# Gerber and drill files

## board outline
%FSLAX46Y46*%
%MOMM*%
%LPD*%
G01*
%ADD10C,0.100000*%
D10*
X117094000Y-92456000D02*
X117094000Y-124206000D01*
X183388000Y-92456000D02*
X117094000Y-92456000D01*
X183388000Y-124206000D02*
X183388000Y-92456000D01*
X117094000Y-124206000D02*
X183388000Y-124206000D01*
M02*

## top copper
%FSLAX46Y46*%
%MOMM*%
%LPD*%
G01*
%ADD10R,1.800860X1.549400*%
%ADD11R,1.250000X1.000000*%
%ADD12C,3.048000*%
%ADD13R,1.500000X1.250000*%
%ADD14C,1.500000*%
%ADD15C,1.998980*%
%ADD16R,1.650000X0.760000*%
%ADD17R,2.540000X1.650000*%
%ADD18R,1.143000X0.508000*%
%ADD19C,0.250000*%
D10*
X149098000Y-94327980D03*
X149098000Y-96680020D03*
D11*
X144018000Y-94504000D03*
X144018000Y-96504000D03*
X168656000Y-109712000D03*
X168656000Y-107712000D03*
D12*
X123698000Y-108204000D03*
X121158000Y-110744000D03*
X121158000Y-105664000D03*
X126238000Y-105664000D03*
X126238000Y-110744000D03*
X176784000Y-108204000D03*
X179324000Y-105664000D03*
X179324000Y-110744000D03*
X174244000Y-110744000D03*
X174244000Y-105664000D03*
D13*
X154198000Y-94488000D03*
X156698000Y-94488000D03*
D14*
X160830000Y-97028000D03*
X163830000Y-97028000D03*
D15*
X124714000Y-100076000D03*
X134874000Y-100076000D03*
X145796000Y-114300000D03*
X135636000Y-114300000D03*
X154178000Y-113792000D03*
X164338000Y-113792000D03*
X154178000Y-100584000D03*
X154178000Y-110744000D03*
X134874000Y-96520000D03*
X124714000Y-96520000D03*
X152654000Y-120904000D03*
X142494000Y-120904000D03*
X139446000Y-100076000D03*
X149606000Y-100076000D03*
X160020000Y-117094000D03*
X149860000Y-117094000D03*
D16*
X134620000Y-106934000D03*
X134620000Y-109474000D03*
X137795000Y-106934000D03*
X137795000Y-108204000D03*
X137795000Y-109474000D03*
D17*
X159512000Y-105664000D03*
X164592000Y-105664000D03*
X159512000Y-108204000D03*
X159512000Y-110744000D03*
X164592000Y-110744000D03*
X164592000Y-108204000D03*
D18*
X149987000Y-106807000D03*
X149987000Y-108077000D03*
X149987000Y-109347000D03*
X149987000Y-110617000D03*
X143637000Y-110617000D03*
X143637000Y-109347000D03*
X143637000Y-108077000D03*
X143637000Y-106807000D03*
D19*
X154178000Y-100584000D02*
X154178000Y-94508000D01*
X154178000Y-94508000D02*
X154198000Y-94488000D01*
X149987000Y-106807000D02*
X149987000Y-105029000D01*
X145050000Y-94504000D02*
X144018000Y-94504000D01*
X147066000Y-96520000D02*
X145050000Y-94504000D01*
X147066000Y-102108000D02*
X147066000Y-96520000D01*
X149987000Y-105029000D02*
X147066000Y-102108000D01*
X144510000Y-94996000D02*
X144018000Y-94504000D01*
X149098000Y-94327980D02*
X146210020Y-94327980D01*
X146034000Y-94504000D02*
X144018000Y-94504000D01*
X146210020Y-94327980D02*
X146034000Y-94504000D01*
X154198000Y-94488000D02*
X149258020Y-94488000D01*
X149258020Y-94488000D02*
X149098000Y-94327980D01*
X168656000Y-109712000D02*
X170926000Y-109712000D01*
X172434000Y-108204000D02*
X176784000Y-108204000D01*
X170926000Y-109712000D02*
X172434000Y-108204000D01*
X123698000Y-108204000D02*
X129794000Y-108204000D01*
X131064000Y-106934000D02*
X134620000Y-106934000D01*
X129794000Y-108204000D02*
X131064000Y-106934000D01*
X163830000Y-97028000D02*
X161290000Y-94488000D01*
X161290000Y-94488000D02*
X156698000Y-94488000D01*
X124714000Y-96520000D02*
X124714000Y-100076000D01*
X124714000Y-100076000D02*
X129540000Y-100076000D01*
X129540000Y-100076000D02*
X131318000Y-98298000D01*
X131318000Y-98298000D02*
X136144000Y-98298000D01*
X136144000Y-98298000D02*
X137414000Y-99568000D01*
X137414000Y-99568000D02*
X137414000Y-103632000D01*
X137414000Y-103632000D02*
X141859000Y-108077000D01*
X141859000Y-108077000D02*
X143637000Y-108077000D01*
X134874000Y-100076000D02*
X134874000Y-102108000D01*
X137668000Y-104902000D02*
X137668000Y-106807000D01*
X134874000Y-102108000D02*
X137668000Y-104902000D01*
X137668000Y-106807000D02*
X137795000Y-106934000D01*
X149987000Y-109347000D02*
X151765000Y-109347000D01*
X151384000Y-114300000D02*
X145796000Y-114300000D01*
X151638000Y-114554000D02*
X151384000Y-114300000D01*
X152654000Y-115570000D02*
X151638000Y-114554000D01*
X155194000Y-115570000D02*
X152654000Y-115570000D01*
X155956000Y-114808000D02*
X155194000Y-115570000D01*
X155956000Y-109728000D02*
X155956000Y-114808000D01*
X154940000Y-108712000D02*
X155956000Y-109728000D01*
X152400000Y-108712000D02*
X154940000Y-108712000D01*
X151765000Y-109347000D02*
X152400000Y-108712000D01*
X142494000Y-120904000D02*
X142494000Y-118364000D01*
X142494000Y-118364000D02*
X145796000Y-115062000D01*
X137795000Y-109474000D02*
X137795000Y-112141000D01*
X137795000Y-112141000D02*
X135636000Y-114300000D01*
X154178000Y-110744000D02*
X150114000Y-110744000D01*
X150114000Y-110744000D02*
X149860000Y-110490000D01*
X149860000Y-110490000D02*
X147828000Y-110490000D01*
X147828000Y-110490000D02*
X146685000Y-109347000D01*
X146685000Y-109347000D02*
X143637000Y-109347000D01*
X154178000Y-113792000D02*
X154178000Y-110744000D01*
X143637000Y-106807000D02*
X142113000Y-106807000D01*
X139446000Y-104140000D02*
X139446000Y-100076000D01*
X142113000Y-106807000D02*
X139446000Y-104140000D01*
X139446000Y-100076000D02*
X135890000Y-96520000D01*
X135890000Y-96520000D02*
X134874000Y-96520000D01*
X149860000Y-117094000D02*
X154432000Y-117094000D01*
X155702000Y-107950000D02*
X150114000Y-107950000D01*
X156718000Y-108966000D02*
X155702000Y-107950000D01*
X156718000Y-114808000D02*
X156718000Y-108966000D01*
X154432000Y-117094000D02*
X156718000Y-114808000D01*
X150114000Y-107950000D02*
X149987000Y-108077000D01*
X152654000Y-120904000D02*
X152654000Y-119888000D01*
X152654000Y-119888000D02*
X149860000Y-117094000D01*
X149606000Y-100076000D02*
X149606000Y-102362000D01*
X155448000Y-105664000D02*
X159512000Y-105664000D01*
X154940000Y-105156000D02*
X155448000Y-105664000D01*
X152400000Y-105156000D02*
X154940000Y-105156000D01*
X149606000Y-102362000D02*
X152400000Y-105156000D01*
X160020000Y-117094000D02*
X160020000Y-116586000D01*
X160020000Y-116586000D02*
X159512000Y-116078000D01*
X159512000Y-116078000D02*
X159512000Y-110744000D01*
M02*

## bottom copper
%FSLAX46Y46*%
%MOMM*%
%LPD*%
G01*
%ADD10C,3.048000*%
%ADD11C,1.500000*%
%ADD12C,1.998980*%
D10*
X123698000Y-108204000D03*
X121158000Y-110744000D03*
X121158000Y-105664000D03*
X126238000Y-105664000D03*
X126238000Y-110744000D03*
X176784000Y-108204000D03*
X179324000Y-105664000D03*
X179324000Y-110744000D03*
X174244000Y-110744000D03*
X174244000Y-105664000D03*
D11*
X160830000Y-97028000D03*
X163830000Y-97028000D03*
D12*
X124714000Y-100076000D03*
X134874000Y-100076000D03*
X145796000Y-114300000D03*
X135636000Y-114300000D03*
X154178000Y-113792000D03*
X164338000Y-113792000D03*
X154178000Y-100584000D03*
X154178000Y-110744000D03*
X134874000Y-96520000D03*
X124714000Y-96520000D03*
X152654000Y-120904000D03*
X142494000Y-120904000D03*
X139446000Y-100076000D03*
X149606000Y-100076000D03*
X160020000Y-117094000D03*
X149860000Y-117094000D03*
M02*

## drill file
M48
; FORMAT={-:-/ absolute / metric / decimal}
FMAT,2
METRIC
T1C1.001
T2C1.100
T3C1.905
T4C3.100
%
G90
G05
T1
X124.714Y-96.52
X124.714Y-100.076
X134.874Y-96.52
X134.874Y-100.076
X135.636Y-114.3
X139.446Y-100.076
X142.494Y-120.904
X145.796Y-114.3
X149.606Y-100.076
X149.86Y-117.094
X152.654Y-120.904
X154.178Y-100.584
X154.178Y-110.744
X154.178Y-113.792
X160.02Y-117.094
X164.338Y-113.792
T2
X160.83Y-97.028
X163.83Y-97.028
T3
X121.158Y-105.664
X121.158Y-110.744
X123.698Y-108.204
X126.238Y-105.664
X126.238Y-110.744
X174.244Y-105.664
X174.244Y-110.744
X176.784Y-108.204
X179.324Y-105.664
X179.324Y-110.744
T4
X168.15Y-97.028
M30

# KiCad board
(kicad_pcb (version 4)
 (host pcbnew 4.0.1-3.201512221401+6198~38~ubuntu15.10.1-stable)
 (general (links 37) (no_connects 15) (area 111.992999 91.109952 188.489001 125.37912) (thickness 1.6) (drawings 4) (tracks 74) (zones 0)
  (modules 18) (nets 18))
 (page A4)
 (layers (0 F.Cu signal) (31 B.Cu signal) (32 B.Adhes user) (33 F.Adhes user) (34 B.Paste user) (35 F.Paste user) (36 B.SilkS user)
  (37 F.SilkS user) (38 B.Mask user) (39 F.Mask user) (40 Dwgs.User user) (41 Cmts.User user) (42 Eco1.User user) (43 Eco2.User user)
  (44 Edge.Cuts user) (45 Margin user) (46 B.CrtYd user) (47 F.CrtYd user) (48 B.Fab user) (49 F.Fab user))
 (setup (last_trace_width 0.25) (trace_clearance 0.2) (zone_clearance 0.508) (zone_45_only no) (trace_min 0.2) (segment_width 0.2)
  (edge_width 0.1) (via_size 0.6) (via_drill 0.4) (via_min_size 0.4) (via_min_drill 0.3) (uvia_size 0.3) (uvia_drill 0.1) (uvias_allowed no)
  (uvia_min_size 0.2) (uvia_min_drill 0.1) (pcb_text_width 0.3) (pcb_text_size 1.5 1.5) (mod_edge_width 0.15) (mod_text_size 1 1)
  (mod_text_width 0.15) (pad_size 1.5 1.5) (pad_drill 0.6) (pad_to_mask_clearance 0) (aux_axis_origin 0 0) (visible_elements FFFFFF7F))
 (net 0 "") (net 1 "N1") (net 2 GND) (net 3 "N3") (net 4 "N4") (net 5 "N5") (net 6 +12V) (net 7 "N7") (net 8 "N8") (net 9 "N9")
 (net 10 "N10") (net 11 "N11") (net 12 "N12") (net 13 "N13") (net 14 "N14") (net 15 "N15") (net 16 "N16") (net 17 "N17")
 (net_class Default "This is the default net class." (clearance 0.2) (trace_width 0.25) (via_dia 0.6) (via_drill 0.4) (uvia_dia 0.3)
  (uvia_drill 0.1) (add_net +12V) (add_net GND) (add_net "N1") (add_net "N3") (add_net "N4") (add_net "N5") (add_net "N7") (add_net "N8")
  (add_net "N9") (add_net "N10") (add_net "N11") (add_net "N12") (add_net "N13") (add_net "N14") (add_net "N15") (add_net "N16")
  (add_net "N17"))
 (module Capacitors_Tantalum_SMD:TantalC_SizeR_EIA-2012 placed (layer F.Cu) (at 149.098 95.504 90)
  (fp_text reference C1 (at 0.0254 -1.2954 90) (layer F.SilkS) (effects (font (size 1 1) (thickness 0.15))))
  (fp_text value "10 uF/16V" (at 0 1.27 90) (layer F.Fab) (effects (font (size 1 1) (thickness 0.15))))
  (pad 1 smd rect (at 1.17602 0 90) (size 1.5494 1.80086) (layers F.Cu F.Paste F.Mask) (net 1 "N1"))
  (pad 2 smd rect (at -1.17602 0 90) (size 1.5494 1.80086) (layers F.Cu F.Paste F.Mask) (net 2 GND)))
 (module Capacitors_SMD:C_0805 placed (layer F.Cu) (at 144.018 95.504 270)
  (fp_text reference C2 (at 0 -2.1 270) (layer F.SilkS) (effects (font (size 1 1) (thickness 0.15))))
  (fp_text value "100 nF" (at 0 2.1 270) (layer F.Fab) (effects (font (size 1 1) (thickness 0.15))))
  (pad 1 smd rect (at -1 0 270) (size 1 1.25) (layers F.Cu F.Paste F.Mask) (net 1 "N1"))
  (pad 2 smd rect (at 1 0 270) (size 1 1.25) (layers F.Cu F.Paste F.Mask) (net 2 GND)))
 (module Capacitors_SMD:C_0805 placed (layer F.Cu) (at 168.656 108.712 90)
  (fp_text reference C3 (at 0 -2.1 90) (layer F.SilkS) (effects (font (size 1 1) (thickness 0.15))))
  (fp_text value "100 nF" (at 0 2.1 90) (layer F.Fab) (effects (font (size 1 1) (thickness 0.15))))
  (pad 1 smd rect (at -1 0 90) (size 1 1.25) (layers F.Cu F.Paste F.Mask) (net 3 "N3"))
  (pad 2 smd rect (at 1 0 90) (size 1 1.25) (layers F.Cu F.Paste F.Mask) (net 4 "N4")))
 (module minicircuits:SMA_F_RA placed (layer F.Cu) (at 123.698 108.204 180)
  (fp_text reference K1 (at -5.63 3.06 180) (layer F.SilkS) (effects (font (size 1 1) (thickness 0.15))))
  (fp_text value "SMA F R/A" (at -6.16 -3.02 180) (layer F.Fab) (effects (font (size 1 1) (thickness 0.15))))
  (pad 1 thru_hole circle (at 0 0 180) (size 3.048 3.048) (drill 1.905) (layers *.Cu *.Mask F.SilkS) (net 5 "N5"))
  (pad 2 thru_hole circle (at 2.54 -2.54 180) (size 3.048 3.048) (drill 1.905) (layers *.Cu *.Mask F.SilkS) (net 2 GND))
  (pad 3 thru_hole circle (at 2.54 2.54 180) (size 3.048 3.048) (drill 1.905) (layers *.Cu *.Mask F.SilkS) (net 2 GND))
  (pad 4 thru_hole circle (at -2.54 2.54 180) (size 3.048 3.048) (drill 1.905) (layers *.Cu *.Mask F.SilkS) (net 2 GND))
  (pad 5 thru_hole circle (at -2.54 -2.54 180) (size 3.048 3.048) (drill 1.905) (layers *.Cu *.Mask F.SilkS) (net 2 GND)))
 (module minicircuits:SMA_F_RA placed (layer F.Cu) (at 176.784 108.204)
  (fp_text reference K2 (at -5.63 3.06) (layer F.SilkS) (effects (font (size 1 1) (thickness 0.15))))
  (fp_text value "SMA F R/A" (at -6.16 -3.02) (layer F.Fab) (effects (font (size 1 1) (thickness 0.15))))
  (pad 1 thru_hole circle (at 0 0) (size 3.048 3.048) (drill 1.905) (layers *.Cu *.Mask F.SilkS) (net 3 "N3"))
  (pad 2 thru_hole circle (at 2.54 -2.54) (size 3.048 3.048) (drill 1.905) (layers *.Cu *.Mask F.SilkS) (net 2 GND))
  (pad 3 thru_hole circle (at 2.54 2.54) (size 3.048 3.048) (drill 1.905) (layers *.Cu *.Mask F.SilkS) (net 2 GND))
  (pad 4 thru_hole circle (at -2.54 2.54) (size 3.048 3.048) (drill 1.905) (layers *.Cu *.Mask F.SilkS) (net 2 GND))
  (pad 5 thru_hole circle (at -2.54 -2.54) (size 3.048 3.048) (drill 1.905) (layers *.Cu *.Mask F.SilkS) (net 2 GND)))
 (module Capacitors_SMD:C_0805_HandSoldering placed (layer F.Cu) (at 155.448 94.488)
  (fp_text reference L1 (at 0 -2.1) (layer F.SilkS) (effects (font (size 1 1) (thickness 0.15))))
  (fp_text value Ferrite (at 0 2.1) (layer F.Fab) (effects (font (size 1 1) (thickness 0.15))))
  (pad 1 smd rect (at -1.25 0) (size 1.5 1.25) (layers F.Cu F.Paste F.Mask) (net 1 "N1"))
  (pad 2 smd rect (at 1.25 0) (size 1.5 1.25) (layers F.Cu F.Paste F.Mask) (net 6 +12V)))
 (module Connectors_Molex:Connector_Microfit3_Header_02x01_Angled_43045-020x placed (layer F.Cu) (at 163.83 97.028 90)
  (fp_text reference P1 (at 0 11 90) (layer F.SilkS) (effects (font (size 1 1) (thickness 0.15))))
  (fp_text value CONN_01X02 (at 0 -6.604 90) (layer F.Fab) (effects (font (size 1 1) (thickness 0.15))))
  (pad 2 thru_hole circle (at 0 -3 90) (size 1.5 1.5) (drill 1.1) (layers *.Cu *.Mask F.SilkS) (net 2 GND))
  (pad 1 thru_hole circle (at 0 0 90) (size 1.5 1.5) (drill 1.1) (layers *.Cu *.Mask F.SilkS) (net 6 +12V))
  (pad "" np_thru_hole circle (at 0 4.32 90) (size 3.1 3.1) (drill 3.1) (layers *.Cu *.Mask F.SilkS)))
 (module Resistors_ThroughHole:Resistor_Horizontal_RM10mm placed (layer F.Cu) (at 129.794 100.076)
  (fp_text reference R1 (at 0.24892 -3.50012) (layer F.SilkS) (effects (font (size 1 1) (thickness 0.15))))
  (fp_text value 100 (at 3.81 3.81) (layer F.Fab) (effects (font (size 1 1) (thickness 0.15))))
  (pad 1 thru_hole circle (at -5.08 0) (size 1.99898 1.99898) (drill 1.00076) (layers *.Cu *.SilkS *.Mask) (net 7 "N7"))
  (pad 2 thru_hole circle (at 5.08 0) (size 1.99898 1.99898) (drill 1.00076) (layers *.Cu *.SilkS *.Mask) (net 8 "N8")))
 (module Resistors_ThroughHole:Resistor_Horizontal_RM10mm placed (layer F.Cu) (at 140.716 114.3 180)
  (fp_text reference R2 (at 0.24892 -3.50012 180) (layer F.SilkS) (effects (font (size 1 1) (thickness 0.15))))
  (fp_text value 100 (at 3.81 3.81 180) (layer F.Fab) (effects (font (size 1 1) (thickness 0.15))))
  (pad 1 thru_hole circle (at -5.08 0 180) (size 1.99898 1.99898) (drill 1.00076) (layers *.Cu *.SilkS *.Mask) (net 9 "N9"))
  (pad 2 thru_hole circle (at 5.08 0 180) (size 1.99898 1.99898) (drill 1.00076) (layers *.Cu *.SilkS *.Mask) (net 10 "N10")))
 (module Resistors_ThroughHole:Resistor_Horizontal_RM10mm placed (layer F.Cu) (at 159.258 113.792)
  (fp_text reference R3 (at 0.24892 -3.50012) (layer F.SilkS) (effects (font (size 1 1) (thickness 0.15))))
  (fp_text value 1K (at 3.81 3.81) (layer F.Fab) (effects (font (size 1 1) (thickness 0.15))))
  (pad 1 thru_hole circle (at -5.08 0) (size 1.99898 1.99898) (drill 1.00076) (layers *.Cu *.SilkS *.Mask) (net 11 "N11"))
  (pad 2 thru_hole circle (at 5.08 0) (size 1.99898 1.99898) (drill 1.00076) (layers *.Cu *.SilkS *.Mask) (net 2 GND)))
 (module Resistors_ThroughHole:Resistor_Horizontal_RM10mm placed (layer F.Cu) (at 154.178 105.664 270)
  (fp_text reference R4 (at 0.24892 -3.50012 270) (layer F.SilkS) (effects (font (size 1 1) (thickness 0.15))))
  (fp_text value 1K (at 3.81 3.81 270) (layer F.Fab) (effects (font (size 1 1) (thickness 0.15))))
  (pad 1 thru_hole circle (at -5.08 0 270) (size 1.99898 1.99898) (drill 1.00076) (layers *.Cu *.SilkS *.Mask) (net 1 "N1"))
  (pad 2 thru_hole circle (at 5.08 0 270) (size 1.99898 1.99898) (drill 1.00076) (layers *.Cu *.SilkS *.Mask) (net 11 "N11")))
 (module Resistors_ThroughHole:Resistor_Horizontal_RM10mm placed (layer F.Cu) (at 129.794 96.52 180)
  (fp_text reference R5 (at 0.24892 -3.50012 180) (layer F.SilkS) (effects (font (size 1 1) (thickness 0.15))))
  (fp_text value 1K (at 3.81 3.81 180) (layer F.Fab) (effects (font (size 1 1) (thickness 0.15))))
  (pad 1 thru_hole circle (at -5.08 0 180) (size 1.99898 1.99898) (drill 1.00076) (layers *.Cu *.SilkS *.Mask) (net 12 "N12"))
  (pad 2 thru_hole circle (at 5.08 0 180) (size 1.99898 1.99898) (drill 1.00076) (layers *.Cu *.SilkS *.Mask) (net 7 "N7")))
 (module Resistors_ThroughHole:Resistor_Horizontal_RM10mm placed (layer F.Cu) (at 147.574 120.904 180)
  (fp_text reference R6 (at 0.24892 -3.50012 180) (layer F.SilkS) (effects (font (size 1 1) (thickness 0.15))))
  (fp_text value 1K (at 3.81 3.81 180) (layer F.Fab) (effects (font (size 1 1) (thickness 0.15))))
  (pad 1 thru_hole circle (at -5.08 0 180) (size 1.99898 1.99898) (drill 1.00076) (layers *.Cu *.SilkS *.Mask) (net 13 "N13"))
  (pad 2 thru_hole circle (at 5.08 0 180) (size 1.99898 1.99898) (drill 1.00076) (layers *.Cu *.SilkS *.Mask) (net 9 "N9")))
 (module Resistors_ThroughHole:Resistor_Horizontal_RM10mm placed (layer F.Cu) (at 144.526 100.076)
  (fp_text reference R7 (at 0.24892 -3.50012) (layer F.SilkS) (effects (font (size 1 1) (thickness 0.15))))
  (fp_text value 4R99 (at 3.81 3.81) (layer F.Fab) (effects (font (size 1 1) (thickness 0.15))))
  (pad 1 thru_hole circle (at -5.08 0) (size 1.99898 1.99898) (drill 1.00076) (layers *.Cu *.SilkS *.Mask) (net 12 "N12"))
  (pad 2 thru_hole circle (at 5.08 0) (size 1.99898 1.99898) (drill 1.00076) (layers *.Cu *.SilkS *.Mask) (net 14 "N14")))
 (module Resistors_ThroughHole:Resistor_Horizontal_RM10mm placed (layer F.Cu) (at 154.94 117.094 180)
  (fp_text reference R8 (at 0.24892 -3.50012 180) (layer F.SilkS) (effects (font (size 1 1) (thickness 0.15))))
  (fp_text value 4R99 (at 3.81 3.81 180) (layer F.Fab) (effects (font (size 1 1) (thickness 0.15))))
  (pad 1 thru_hole circle (at -5.08 0 180) (size 1.99898 1.99898) (drill 1.00076) (layers *.Cu *.SilkS *.Mask) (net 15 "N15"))
  (pad 2 thru_hole circle (at 5.08 0 180) (size 1.99898 1.99898) (drill 1.00076) (layers *.Cu *.SilkS *.Mask) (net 13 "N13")))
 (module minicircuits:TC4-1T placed (layer F.Cu) (at 134.62 106.934 270)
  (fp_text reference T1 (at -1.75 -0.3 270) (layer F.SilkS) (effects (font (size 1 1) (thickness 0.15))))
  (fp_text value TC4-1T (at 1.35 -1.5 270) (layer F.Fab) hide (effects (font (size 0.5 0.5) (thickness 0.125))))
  (pad 5 smd rect (at 0 0 270) (size 0.76 1.65) (layers F.Cu F.Paste F.Mask) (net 5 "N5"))
  (pad 4 smd rect (at 2.54 0 270) (size 0.76 1.65) (layers F.Cu F.Paste F.Mask) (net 2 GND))
  (pad 1 smd rect (at 0 -3.175 270) (size 0.76 1.65) (layers F.Cu F.Paste F.Mask) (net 8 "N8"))
  (pad 2 smd rect (at 1.27 -3.175 270) (size 0.76 1.65) (layers F.Cu F.Paste F.Mask) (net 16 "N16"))
  (pad 3 smd rect (at 2.54 -3.175 270) (size 0.76 1.65) (layers F.Cu F.Paste F.Mask) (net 10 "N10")))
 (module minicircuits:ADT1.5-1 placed (layer F.Cu) (at 159.512 105.664 270)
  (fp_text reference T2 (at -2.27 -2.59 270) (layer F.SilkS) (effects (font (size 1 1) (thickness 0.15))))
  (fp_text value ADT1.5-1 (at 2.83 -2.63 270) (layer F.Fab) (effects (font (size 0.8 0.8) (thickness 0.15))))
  (pad 1 smd rect (at 0 0 270) (size 1.65 2.54) (layers F.Cu F.Paste F.Mask) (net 14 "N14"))
  (pad 6 smd rect (at 0 -5.08 270) (size 1.65 2.54) (layers F.Cu F.Paste F.Mask))
  (pad 2 smd rect (at 2.54 0 270) (size 1.65 2.54) (layers F.Cu F.Paste F.Mask) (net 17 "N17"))
  (pad 3 smd rect (at 5.08 0 270) (size 1.65 2.54) (layers F.Cu F.Paste F.Mask) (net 15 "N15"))
  (pad 4 smd rect (at 5.08 -5.08 270) (size 1.65 2.54) (layers F.Cu F.Paste F.Mask) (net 2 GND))
  (pad 5 smd rect (at 2.54 -5.08 270) (size 1.65 2.54) (layers F.Cu F.Paste F.Mask) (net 4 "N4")))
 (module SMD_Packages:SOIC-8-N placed (layer F.Cu) (at 146.812 108.712 270)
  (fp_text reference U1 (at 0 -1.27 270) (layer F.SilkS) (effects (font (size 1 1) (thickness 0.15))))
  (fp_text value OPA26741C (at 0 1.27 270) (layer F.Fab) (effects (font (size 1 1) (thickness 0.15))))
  (pad 8 smd rect (at -1.905 -3.175 270) (size 0.508 1.143) (layers F.Cu F.Paste F.Mask) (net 1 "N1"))
  (pad 7 smd rect (at -0.635 -3.175 270) (size 0.508 1.143) (layers F.Cu F.Paste F.Mask) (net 13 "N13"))
  (pad 6 smd rect (at 0.635 -3.175 270) (size 0.508 1.143) (layers F.Cu F.Paste F.Mask) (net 9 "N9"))
  (pad 5 smd rect (at 1.905 -3.175 270) (size 0.508 1.143) (layers F.Cu F.Paste F.Mask) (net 11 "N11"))
  (pad 4 smd rect (at 1.905 3.175 270) (size 0.508 1.143) (layers F.Cu F.Paste F.Mask) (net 2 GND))
  (pad 3 smd rect (at 0.635 3.175 270) (size 0.508 1.143) (layers F.Cu F.Paste F.Mask) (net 11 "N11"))
  (pad 2 smd rect (at -0.635 3.175 270) (size 0.508 1.143) (layers F.Cu F.Paste F.Mask) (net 7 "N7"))
  (pad 1 smd rect (at -1.905 3.175 270) (size 0.508 1.143) (layers F.Cu F.Paste F.Mask) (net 12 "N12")))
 (gr_line (start 117.094 92.456) (end 117.094 124.206) (angle 90) (layer Edge.Cuts) (width 0.1))
 (gr_line (start 183.388 92.456) (end 117.094 92.456) (angle 90) (layer Edge.Cuts) (width 0.1))
 (gr_line (start 183.388 124.206) (end 183.388 92.456) (angle 90) (layer Edge.Cuts) (width 0.1))
 (gr_line (start 117.094 124.206) (end 183.388 124.206) (angle 90) (layer Edge.Cuts) (width 0.1))
 (segment (start 154.178 100.584) (end 154.178 94.508) (width 0.25) (layer F.Cu) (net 1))
 (segment (start 154.178 94.508) (end 154.198 94.488) (width 0.25) (layer F.Cu) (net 1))
 (segment (start 149.987 106.807) (end 149.987 105.029) (width 0.25) (layer F.Cu) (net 1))
 (segment (start 145.05 94.504) (end 144.018 94.504) (width 0.25) (layer F.Cu) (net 1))
 (segment (start 147.066 96.52) (end 145.05 94.504) (width 0.25) (layer F.Cu) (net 1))
 (segment (start 147.066 102.108) (end 147.066 96.52) (width 0.25) (layer F.Cu) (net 1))
 (segment (start 149.987 105.029) (end 147.066 102.108) (width 0.25) (layer F.Cu) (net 1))
 (segment (start 144.51 94.996) (end 144.018 94.504) (width 0.25) (layer F.Cu) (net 1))
 (segment (start 149.098 94.32798) (end 146.21002 94.32798) (width 0.25) (layer F.Cu) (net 1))
 (segment (start 146.034 94.504) (end 144.018 94.504) (width 0.25) (layer F.Cu) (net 1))
 (segment (start 146.21002 94.32798) (end 146.034 94.504) (width 0.25) (layer F.Cu) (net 1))
 (segment (start 154.198 94.488) (end 149.25802 94.488) (width 0.25) (layer F.Cu) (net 1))
 (segment (start 149.25802 94.488) (end 149.098 94.32798) (width 0.25) (layer F.Cu) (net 1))
 (segment (start 168.656 109.712) (end 170.926 109.712) (width 0.25) (layer F.Cu) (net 3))
 (segment (start 172.434 108.204) (end 176.784 108.204) (width 0.25) (layer F.Cu) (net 3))
 (segment (start 170.926 109.712) (end 172.434 108.204) (width 0.25) (layer F.Cu) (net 3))
 (segment (start 123.698 108.204) (end 129.794 108.204) (width 0.25) (layer F.Cu) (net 5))
 (segment (start 131.064 106.934) (end 134.62 106.934) (width 0.25) (layer F.Cu) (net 5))
 (segment (start 129.794 108.204) (end 131.064 106.934) (width 0.25) (layer F.Cu) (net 5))
 (segment (start 163.83 97.028) (end 161.29 94.488) (width 0.25) (layer F.Cu) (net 6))
 (segment (start 161.29 94.488) (end 156.698 94.488) (width 0.25) (layer F.Cu) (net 6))
 (segment (start 124.714 96.52) (end 124.714 100.076) (width 0.25) (layer F.Cu) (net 7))
 (segment (start 124.714 100.076) (end 129.54 100.076) (width 0.25) (layer F.Cu) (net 7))
 (segment (start 129.54 100.076) (end 131.318 98.298) (width 0.25) (layer F.Cu) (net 7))
 (segment (start 131.318 98.298) (end 136.144 98.298) (width 0.25) (layer F.Cu) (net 7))
 (segment (start 136.144 98.298) (end 137.414 99.568) (width 0.25) (layer F.Cu) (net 7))
 (segment (start 137.414 99.568) (end 137.414 103.632) (width 0.25) (layer F.Cu) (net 7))
 (segment (start 137.414 103.632) (end 141.859 108.077) (width 0.25) (layer F.Cu) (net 7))
 (segment (start 141.859 108.077) (end 143.637 108.077) (width 0.25) (layer F.Cu) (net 7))
 (segment (start 134.874 100.076) (end 134.874 102.108) (width 0.25) (layer F.Cu) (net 8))
 (segment (start 137.668 104.902) (end 137.668 106.807) (width 0.25) (layer F.Cu) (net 8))
 (segment (start 134.874 102.108) (end 137.668 104.902) (width 0.25) (layer F.Cu) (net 8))
 (segment (start 137.668 106.807) (end 137.795 106.934) (width 0.25) (layer F.Cu) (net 8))
 (segment (start 149.987 109.347) (end 151.765 109.347) (width 0.25) (layer F.Cu) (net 9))
 (segment (start 151.384 114.3) (end 145.796 114.3) (width 0.25) (layer F.Cu) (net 9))
 (segment (start 151.638 114.554) (end 151.384 114.3) (width 0.25) (layer F.Cu) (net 9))
 (segment (start 152.654 115.57) (end 151.638 114.554) (width 0.25) (layer F.Cu) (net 9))
 (segment (start 155.194 115.57) (end 152.654 115.57) (width 0.25) (layer F.Cu) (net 9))
 (segment (start 155.956 114.808) (end 155.194 115.57) (width 0.25) (layer F.Cu) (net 9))
 (segment (start 155.956 109.728) (end 155.956 114.808) (width 0.25) (layer F.Cu) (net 9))
 (segment (start 154.94 108.712) (end 155.956 109.728) (width 0.25) (layer F.Cu) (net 9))
 (segment (start 152.4 108.712) (end 154.94 108.712) (width 0.25) (layer F.Cu) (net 9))
 (segment (start 151.765 109.347) (end 152.4 108.712) (width 0.25) (layer F.Cu) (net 9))
 (segment (start 142.494 120.904) (end 142.494 118.364) (width 0.25) (layer F.Cu) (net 9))
 (segment (start 142.494 118.364) (end 145.796 115.062) (width 0.25) (layer F.Cu) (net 9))
 (segment (start 137.795 109.474) (end 137.795 112.141) (width 0.25) (layer F.Cu) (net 10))
 (segment (start 137.795 112.141) (end 135.636 114.3) (width 0.25) (layer F.Cu) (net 10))
 (segment (start 154.178 110.744) (end 150.114 110.744) (width 0.25) (layer F.Cu) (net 11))
 (segment (start 150.114 110.744) (end 149.86 110.49) (width 0.25) (layer F.Cu) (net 11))
 (segment (start 149.86 110.49) (end 147.828 110.49) (width 0.25) (layer F.Cu) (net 11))
 (segment (start 147.828 110.49) (end 146.685 109.347) (width 0.25) (layer F.Cu) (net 11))
 (segment (start 146.685 109.347) (end 143.637 109.347) (width 0.25) (layer F.Cu) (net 11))
 (segment (start 154.178 113.792) (end 154.178 110.744) (width 0.25) (layer F.Cu) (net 11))
 (segment (start 143.637 106.807) (end 142.113 106.807) (width 0.25) (layer F.Cu) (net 12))
 (segment (start 139.446 104.14) (end 139.446 100.076) (width 0.25) (layer F.Cu) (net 12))
 (segment (start 142.113 106.807) (end 139.446 104.14) (width 0.25) (layer F.Cu) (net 12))
 (segment (start 139.446 100.076) (end 135.89 96.52) (width 0.25) (layer F.Cu) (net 12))
 (segment (start 135.89 96.52) (end 134.874 96.52) (width 0.25) (layer F.Cu) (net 12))
 (segment (start 149.86 117.094) (end 154.432 117.094) (width 0.25) (layer F.Cu) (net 13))
 (segment (start 155.702 107.95) (end 150.114 107.95) (width 0.25) (layer F.Cu) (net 13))
 (segment (start 156.718 108.966) (end 155.702 107.95) (width 0.25) (layer F.Cu) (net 13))
 (segment (start 156.718 114.808) (end 156.718 108.966) (width 0.25) (layer F.Cu) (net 13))
 (segment (start 154.432 117.094) (end 156.718 114.808) (width 0.25) (layer F.Cu) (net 13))
 (segment (start 150.114 107.95) (end 149.987 108.077) (width 0.25) (layer F.Cu) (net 13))
 (segment (start 152.654 120.904) (end 152.654 119.888) (width 0.25) (layer F.Cu) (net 13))
 (segment (start 152.654 119.888) (end 149.86 117.094) (width 0.25) (layer F.Cu) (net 13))
 (segment (start 149.606 100.076) (end 149.606 102.362) (width 0.25) (layer F.Cu) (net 14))
 (segment (start 155.448 105.664) (end 159.512 105.664) (width 0.25) (layer F.Cu) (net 14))
 (segment (start 154.94 105.156) (end 155.448 105.664) (width 0.25) (layer F.Cu) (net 14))
 (segment (start 152.4 105.156) (end 154.94 105.156) (width 0.25) (layer F.Cu) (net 14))
 (segment (start 149.606 102.362) (end 152.4 105.156) (width 0.25) (layer F.Cu) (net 14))
 (segment (start 160.02 117.094) (end 160.02 116.586) (width 0.25) (layer F.Cu) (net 15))
 (segment (start 160.02 116.586) (end 159.512 116.078) (width 0.25) (layer F.Cu) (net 15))
 (segment (start 159.512 116.078) (end 159.512 110.744) (width 0.25) (layer F.Cu) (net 15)))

